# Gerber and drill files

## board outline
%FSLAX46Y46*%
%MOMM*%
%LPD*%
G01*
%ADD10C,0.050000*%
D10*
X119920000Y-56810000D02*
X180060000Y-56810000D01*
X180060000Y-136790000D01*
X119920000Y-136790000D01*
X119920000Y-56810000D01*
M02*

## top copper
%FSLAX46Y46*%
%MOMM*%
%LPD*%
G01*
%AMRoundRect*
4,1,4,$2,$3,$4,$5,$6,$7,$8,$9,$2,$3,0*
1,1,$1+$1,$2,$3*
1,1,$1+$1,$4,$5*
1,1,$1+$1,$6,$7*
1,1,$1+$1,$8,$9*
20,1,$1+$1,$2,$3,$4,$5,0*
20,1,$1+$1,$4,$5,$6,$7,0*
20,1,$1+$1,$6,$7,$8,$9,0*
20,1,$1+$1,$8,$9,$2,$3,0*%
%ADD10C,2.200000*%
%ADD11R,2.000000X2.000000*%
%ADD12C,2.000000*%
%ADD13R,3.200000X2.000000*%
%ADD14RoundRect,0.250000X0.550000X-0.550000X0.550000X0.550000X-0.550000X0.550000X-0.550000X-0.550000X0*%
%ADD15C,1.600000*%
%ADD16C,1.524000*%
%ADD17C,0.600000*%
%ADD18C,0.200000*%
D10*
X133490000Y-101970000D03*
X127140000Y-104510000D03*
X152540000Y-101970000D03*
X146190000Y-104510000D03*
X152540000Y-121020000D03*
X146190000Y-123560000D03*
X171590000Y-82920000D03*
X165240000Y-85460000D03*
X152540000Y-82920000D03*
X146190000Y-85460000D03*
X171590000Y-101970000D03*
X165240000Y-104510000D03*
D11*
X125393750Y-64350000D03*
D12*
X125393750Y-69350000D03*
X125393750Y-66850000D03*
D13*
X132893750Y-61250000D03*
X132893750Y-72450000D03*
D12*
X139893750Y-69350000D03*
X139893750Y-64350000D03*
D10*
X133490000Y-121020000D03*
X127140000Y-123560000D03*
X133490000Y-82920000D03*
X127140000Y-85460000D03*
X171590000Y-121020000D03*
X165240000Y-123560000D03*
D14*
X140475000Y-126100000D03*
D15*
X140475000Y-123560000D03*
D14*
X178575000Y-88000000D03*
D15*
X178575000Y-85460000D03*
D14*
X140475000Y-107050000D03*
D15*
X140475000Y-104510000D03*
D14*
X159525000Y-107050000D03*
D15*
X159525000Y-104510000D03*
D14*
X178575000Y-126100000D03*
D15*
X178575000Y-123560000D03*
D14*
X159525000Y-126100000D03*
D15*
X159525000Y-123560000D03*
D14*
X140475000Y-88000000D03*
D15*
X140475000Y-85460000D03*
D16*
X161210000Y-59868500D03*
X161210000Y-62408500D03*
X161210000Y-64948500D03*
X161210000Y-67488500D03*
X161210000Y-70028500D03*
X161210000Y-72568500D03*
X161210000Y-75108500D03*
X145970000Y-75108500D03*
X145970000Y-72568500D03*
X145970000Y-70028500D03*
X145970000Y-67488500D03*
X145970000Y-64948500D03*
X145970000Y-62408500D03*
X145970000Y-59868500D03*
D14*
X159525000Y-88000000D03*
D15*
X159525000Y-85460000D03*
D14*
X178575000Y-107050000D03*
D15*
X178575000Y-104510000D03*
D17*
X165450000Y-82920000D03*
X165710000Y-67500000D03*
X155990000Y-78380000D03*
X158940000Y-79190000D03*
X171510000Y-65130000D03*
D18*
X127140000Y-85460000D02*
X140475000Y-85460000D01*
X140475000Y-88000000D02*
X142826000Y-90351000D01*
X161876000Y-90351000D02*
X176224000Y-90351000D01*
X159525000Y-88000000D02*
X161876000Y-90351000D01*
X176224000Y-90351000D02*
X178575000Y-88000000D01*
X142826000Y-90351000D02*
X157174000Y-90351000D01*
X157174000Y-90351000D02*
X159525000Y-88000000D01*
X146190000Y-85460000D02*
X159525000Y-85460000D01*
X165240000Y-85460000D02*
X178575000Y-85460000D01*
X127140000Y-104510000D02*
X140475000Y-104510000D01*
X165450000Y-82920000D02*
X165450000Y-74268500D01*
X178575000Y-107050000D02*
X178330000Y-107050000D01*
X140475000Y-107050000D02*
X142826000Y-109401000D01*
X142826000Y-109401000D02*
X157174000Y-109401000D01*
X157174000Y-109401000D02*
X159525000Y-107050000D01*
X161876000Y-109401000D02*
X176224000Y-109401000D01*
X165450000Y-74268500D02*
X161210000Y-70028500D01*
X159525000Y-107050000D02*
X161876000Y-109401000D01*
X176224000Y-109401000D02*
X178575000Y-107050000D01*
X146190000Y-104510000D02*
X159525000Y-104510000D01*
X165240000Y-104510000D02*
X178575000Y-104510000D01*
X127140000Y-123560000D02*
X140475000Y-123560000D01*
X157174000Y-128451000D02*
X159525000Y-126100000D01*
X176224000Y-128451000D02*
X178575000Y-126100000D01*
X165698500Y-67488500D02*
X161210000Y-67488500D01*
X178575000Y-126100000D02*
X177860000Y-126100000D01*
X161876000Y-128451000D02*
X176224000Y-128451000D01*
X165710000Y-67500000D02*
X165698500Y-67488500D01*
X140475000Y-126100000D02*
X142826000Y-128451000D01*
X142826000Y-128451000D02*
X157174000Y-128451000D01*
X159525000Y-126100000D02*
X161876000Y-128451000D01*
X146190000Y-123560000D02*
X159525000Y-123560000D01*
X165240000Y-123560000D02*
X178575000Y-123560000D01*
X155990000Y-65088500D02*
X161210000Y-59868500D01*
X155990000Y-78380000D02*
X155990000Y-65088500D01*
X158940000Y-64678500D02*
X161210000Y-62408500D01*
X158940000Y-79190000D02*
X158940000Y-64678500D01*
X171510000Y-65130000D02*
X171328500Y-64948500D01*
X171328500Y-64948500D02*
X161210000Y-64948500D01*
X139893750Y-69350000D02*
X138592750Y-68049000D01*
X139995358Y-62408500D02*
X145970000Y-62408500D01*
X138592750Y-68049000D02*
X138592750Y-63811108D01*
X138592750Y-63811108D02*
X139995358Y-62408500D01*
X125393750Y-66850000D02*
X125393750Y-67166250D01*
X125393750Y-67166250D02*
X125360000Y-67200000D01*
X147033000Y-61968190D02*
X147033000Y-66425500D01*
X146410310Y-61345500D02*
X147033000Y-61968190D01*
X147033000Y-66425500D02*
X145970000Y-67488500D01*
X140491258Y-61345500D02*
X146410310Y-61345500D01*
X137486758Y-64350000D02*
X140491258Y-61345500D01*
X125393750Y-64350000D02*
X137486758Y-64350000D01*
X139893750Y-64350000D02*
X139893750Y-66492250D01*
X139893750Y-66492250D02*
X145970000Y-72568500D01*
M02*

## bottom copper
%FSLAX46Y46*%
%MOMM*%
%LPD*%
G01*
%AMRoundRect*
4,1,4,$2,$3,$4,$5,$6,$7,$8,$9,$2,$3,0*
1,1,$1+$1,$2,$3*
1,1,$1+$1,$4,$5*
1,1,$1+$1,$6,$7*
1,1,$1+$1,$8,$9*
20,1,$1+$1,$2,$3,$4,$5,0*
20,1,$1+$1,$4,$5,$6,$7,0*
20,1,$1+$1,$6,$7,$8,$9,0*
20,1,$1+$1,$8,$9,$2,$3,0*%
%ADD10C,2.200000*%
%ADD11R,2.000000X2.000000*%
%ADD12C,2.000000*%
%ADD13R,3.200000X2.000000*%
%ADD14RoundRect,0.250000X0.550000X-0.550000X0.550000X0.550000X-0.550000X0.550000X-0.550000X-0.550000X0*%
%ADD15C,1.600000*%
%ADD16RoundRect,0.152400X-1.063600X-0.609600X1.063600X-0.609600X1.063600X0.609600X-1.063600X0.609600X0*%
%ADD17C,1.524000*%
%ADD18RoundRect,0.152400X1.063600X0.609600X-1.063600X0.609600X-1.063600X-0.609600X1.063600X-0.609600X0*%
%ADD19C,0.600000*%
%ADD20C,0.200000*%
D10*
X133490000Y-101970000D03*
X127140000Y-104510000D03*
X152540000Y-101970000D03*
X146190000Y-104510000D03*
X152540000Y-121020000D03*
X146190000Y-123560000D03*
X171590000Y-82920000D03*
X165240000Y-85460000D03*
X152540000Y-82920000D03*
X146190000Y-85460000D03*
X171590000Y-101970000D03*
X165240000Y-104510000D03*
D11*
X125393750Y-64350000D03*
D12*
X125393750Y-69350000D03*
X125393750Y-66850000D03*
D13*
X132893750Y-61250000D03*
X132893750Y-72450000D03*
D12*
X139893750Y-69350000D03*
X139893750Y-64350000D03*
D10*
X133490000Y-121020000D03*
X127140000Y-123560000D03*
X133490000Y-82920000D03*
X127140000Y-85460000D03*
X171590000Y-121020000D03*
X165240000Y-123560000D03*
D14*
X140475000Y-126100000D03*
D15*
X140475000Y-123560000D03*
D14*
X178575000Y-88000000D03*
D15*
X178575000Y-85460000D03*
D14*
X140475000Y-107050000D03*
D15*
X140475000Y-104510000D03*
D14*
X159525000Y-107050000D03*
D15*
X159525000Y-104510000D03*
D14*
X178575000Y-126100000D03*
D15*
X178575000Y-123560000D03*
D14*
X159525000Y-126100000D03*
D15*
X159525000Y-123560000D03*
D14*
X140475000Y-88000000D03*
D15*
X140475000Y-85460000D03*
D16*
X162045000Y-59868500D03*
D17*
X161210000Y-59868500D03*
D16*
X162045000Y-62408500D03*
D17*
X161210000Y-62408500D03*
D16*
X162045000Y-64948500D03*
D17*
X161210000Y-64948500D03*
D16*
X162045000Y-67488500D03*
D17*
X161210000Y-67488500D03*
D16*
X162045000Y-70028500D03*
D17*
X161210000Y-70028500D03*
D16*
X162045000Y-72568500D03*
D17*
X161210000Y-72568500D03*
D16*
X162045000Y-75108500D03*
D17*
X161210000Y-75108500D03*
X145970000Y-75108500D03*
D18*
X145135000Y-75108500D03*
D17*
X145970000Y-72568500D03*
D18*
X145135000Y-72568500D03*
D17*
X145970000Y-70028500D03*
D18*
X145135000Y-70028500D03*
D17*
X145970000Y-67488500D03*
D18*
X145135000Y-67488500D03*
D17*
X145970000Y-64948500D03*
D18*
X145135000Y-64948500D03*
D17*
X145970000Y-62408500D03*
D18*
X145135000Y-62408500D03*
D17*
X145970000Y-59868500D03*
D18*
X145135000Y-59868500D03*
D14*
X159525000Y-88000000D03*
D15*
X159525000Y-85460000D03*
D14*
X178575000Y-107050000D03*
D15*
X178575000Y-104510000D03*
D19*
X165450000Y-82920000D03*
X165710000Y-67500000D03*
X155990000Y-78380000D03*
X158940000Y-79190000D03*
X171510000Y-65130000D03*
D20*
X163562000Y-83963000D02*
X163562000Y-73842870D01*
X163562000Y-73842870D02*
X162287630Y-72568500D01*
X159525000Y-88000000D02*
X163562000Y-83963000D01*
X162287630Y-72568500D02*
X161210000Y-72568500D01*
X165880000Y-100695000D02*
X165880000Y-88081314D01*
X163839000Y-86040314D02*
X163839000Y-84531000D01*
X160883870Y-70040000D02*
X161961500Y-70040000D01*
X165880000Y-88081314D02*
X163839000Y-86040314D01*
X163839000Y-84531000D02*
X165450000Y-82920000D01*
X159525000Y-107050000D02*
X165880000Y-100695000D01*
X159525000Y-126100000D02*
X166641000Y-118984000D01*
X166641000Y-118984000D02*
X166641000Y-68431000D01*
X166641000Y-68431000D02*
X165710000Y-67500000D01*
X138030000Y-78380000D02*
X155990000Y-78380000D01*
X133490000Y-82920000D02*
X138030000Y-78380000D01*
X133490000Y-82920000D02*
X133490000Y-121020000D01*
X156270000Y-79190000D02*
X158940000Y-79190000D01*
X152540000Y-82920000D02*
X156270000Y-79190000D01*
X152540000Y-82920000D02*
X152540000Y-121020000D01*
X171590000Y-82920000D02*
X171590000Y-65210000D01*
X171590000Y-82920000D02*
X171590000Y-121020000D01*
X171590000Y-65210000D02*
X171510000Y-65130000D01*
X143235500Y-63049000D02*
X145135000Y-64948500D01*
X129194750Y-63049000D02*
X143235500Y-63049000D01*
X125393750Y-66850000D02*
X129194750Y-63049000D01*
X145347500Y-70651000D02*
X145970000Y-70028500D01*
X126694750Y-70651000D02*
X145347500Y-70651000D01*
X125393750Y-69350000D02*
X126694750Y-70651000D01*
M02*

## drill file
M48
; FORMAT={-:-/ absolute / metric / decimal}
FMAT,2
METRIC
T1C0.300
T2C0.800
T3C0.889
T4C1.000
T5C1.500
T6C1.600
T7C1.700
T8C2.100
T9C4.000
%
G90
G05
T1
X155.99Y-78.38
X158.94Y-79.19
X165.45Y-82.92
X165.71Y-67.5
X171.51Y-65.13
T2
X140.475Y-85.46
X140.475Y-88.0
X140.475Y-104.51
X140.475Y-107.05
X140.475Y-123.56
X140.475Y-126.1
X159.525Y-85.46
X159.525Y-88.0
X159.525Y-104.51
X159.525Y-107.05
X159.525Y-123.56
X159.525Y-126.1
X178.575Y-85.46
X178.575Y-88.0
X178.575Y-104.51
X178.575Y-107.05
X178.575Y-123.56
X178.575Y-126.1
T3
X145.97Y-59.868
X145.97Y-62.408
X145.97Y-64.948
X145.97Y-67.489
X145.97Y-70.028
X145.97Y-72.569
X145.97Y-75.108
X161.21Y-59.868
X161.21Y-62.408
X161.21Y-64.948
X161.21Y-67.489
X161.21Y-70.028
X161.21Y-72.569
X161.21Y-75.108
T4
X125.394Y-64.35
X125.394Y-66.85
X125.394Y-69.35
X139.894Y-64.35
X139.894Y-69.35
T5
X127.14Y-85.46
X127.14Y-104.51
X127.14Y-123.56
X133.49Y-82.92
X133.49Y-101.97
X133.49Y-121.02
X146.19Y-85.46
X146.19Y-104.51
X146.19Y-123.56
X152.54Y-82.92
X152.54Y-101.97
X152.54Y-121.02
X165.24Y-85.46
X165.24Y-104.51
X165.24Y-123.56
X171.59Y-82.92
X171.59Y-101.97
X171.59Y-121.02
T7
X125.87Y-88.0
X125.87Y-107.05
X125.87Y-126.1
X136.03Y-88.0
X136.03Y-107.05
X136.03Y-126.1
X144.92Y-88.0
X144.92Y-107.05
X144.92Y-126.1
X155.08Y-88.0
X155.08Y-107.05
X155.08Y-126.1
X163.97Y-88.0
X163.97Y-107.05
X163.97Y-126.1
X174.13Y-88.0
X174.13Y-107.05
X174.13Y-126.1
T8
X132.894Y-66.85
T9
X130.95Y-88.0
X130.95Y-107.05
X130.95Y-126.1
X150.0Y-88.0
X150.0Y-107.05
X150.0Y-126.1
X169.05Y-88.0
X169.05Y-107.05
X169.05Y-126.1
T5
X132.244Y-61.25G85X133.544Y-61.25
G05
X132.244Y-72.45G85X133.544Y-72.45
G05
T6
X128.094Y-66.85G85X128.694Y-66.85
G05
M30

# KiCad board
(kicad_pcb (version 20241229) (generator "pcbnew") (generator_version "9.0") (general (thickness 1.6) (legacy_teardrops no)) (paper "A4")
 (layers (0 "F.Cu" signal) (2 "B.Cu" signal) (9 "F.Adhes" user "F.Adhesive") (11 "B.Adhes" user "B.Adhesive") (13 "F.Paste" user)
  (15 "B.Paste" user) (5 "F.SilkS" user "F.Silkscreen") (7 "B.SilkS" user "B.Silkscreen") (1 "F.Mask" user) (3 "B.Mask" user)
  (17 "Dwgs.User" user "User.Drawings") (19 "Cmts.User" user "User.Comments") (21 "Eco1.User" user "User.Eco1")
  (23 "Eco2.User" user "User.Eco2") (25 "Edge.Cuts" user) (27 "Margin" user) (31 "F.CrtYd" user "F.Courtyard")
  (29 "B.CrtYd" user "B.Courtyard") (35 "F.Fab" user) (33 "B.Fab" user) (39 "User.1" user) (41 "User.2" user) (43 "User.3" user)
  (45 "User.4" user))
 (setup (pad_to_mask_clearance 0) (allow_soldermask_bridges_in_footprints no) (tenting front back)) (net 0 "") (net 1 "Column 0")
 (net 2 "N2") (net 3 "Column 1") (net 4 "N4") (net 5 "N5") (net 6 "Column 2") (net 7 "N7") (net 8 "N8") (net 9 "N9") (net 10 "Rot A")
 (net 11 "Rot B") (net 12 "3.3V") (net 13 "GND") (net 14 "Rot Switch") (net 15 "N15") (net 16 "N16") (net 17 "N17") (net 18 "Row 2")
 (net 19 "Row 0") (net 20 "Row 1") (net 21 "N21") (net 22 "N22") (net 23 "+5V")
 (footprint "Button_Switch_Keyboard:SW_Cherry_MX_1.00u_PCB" (layer "F.Cu") (at 133.49 101.97)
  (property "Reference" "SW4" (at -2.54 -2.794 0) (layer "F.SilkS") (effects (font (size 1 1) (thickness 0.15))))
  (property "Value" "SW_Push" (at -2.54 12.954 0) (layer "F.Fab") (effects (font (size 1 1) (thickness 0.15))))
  (pad "" np_thru_hole circle (at -7.62 5.08) (size 1.7 1.7) (drill 1.7) (layers "*.Cu" "*.Mask"))
  (pad "" np_thru_hole circle (at -2.54 5.08) (size 4 4) (drill 4) (layers "*.Cu" "*.Mask"))
  (pad "" np_thru_hole circle (at 2.54 5.08) (size 1.7 1.7) (drill 1.7) (layers "*.Cu" "*.Mask"))
  (pad "1" thru_hole circle (at 0 0) (size 2.2 2.2) (drill 1.5) (layers "*.Cu" "*.Mask") (remove_unused_layers no) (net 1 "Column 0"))
  (pad "2" thru_hole circle (at -6.35 2.54) (size 2.2 2.2) (drill 1.5) (layers "*.Cu" "*.Mask") (remove_unused_layers no) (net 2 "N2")))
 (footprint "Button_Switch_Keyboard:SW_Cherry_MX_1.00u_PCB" (layer "F.Cu") (at 152.54 101.97)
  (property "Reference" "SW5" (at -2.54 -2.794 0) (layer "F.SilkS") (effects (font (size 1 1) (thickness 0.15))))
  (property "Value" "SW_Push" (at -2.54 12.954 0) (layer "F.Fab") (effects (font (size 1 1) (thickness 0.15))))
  (pad "" np_thru_hole circle (at -7.62 5.08) (size 1.7 1.7) (drill 1.7) (layers "*.Cu" "*.Mask"))
  (pad "" np_thru_hole circle (at -2.54 5.08) (size 4 4) (drill 4) (layers "*.Cu" "*.Mask"))
  (pad "" np_thru_hole circle (at 2.54 5.08) (size 1.7 1.7) (drill 1.7) (layers "*.Cu" "*.Mask"))
  (pad "1" thru_hole circle (at 0 0) (size 2.2 2.2) (drill 1.5) (layers "*.Cu" "*.Mask") (remove_unused_layers no) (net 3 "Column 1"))
  (pad "2" thru_hole circle (at -6.35 2.54) (size 2.2 2.2) (drill 1.5) (layers "*.Cu" "*.Mask") (remove_unused_layers no) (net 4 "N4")))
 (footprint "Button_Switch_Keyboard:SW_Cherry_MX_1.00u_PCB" (layer "F.Cu") (at 152.54 121.02)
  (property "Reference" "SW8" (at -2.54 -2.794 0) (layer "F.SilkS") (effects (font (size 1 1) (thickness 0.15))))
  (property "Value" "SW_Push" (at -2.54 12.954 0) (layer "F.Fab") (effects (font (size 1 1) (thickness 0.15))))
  (pad "" np_thru_hole circle (at -7.62 5.08) (size 1.7 1.7) (drill 1.7) (layers "*.Cu" "*.Mask"))
  (pad "" np_thru_hole circle (at -2.54 5.08) (size 4 4) (drill 4) (layers "*.Cu" "*.Mask"))
  (pad "" np_thru_hole circle (at 2.54 5.08) (size 1.7 1.7) (drill 1.7) (layers "*.Cu" "*.Mask"))
  (pad "1" thru_hole circle (at 0 0) (size 2.2 2.2) (drill 1.5) (layers "*.Cu" "*.Mask") (remove_unused_layers no) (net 3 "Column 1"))
  (pad "2" thru_hole circle (at -6.35 2.54) (size 2.2 2.2) (drill 1.5) (layers "*.Cu" "*.Mask") (remove_unused_layers no) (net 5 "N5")))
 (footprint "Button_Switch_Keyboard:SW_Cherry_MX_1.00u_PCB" (layer "F.Cu") (at 171.59 82.92)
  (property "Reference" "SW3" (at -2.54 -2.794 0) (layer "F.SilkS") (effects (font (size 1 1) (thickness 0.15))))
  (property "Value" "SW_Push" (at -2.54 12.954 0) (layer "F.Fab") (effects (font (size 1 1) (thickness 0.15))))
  (pad "" np_thru_hole circle (at -7.62 5.08) (size 1.7 1.7) (drill 1.7) (layers "*.Cu" "*.Mask"))
  (pad "" np_thru_hole circle (at -2.54 5.08) (size 4 4) (drill 4) (layers "*.Cu" "*.Mask"))
  (pad "" np_thru_hole circle (at 2.54 5.08) (size 1.7 1.7) (drill 1.7) (layers "*.Cu" "*.Mask"))
  (pad "1" thru_hole circle (at 0 0) (size 2.2 2.2) (drill 1.5) (layers "*.Cu" "*.Mask") (remove_unused_layers no) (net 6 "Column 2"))
  (pad "2" thru_hole circle (at -6.35 2.54) (size 2.2 2.2) (drill 1.5) (layers "*.Cu" "*.Mask") (remove_unused_layers no) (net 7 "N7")))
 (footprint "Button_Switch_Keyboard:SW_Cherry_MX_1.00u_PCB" (layer "F.Cu") (at 152.54 82.92)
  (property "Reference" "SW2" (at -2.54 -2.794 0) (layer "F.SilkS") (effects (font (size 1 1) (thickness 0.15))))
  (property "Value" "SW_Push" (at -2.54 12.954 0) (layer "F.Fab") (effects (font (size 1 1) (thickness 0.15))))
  (pad "" np_thru_hole circle (at -7.62 5.08) (size 1.7 1.7) (drill 1.7) (layers "*.Cu" "*.Mask"))
  (pad "" np_thru_hole circle (at -2.54 5.08) (size 4 4) (drill 4) (layers "*.Cu" "*.Mask"))
  (pad "" np_thru_hole circle (at 2.54 5.08) (size 1.7 1.7) (drill 1.7) (layers "*.Cu" "*.Mask"))
  (pad "1" thru_hole circle (at 0 0) (size 2.2 2.2) (drill 1.5) (layers "*.Cu" "*.Mask") (remove_unused_layers no) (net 3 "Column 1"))
  (pad "2" thru_hole circle (at -6.35 2.54) (size 2.2 2.2) (drill 1.5) (layers "*.Cu" "*.Mask") (remove_unused_layers no) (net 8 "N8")))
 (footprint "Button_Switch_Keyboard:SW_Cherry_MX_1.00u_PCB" (layer "F.Cu") (at 171.59 101.97)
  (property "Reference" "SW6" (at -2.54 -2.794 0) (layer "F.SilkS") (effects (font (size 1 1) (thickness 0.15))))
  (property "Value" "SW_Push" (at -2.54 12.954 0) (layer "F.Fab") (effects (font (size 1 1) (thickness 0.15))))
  (pad "" np_thru_hole circle (at -7.62 5.08) (size 1.7 1.7) (drill 1.7) (layers "*.Cu" "*.Mask"))
  (pad "" np_thru_hole circle (at -2.54 5.08) (size 4 4) (drill 4) (layers "*.Cu" "*.Mask"))
  (pad "" np_thru_hole circle (at 2.54 5.08) (size 1.7 1.7) (drill 1.7) (layers "*.Cu" "*.Mask"))
  (pad "1" thru_hole circle (at 0 0) (size 2.2 2.2) (drill 1.5) (layers "*.Cu" "*.Mask") (remove_unused_layers no) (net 6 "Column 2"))
  (pad "2" thru_hole circle (at -6.35 2.54) (size 2.2 2.2) (drill 1.5) (layers "*.Cu" "*.Mask") (remove_unused_layers no) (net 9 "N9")))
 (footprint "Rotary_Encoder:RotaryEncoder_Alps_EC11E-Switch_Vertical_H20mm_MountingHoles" (layer "F.Cu") (at 125.39375 64.35)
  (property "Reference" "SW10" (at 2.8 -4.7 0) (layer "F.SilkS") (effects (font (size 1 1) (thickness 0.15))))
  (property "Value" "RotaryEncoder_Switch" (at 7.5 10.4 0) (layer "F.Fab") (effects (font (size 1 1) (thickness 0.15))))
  (pad "" np_thru_hole oval (at 3 2.5) (size 2.2 1.6) (drill oval 2.2 1.6) (layers "*.Mask"))
  (pad "" np_thru_hole circle (at 7.5 2.5) (size 2.1 2.1) (drill 2.1) (layers "*.Mask"))
  (pad "A" thru_hole rect (at 0 0) (size 2 2) (drill 1) (layers "*.Cu" "*.Mask") (remove_unused_layers no) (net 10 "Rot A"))
  (pad "B" thru_hole circle (at 0 5) (size 2 2) (drill 1) (layers "*.Cu" "*.Mask") (remove_unused_layers no) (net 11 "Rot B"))
  (pad "C" thru_hole circle (at 0 2.5) (size 2 2) (drill 1) (layers "*.Cu" "*.Mask") (remove_unused_layers no) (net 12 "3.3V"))
  (pad "MP" thru_hole rect (at 7.5 -3.1) (size 3.2 2) (drill oval 2.8 1.5) (layers "*.Cu" "*.Mask") (remove_unused_layers no))
  (pad "MP" thru_hole rect (at 7.5 8.1) (size 3.2 2) (drill oval 2.8 1.5) (layers "*.Cu" "*.Mask") (remove_unused_layers no))
  (pad "S1" thru_hole circle (at 14.5 5) (size 2 2) (drill 1) (layers "*.Cu" "*.Mask") (remove_unused_layers no) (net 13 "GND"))
  (pad "S2" thru_hole circle (at 14.5 0) (size 2 2) (drill 1) (layers "*.Cu" "*.Mask") (remove_unused_layers no) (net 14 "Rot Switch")))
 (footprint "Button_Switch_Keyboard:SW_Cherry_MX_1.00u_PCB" (layer "F.Cu") (at 133.49 121.02)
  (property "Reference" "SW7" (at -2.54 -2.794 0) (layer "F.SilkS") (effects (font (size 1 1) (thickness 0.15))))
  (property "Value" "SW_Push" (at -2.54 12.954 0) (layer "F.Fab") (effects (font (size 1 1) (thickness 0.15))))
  (pad "" np_thru_hole circle (at -7.62 5.08) (size 1.7 1.7) (drill 1.7) (layers "*.Cu" "*.Mask"))
  (pad "" np_thru_hole circle (at -2.54 5.08) (size 4 4) (drill 4) (layers "*.Cu" "*.Mask"))
  (pad "" np_thru_hole circle (at 2.54 5.08) (size 1.7 1.7) (drill 1.7) (layers "*.Cu" "*.Mask"))
  (pad "1" thru_hole circle (at 0 0) (size 2.2 2.2) (drill 1.5) (layers "*.Cu" "*.Mask") (remove_unused_layers no) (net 1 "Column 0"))
  (pad "2" thru_hole circle (at -6.35 2.54) (size 2.2 2.2) (drill 1.5) (layers "*.Cu" "*.Mask") (remove_unused_layers no) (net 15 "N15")))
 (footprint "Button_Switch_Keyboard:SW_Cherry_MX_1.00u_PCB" (layer "F.Cu") (at 133.49 82.92)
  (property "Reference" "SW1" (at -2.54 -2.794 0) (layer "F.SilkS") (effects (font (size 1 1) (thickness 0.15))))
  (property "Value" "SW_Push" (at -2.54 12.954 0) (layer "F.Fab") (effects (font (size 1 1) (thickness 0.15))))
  (pad "" np_thru_hole circle (at -7.62 5.08) (size 1.7 1.7) (drill 1.7) (layers "*.Cu" "*.Mask"))
  (pad "" np_thru_hole circle (at -2.54 5.08) (size 4 4) (drill 4) (layers "*.Cu" "*.Mask"))
  (pad "" np_thru_hole circle (at 2.54 5.08) (size 1.7 1.7) (drill 1.7) (layers "*.Cu" "*.Mask"))
  (pad "1" thru_hole circle (at 0 0) (size 2.2 2.2) (drill 1.5) (layers "*.Cu" "*.Mask") (remove_unused_layers no) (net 1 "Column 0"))
  (pad "2" thru_hole circle (at -6.35 2.54) (size 2.2 2.2) (drill 1.5) (layers "*.Cu" "*.Mask") (remove_unused_layers no) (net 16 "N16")))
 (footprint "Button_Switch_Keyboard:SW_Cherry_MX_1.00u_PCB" (layer "F.Cu") (at 171.59 121.02)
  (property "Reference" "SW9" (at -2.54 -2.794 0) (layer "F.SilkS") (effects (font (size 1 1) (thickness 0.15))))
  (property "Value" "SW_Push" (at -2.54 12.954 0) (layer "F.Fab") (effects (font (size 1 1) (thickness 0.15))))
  (pad "" np_thru_hole circle (at -7.62 5.08) (size 1.7 1.7) (drill 1.7) (layers "*.Cu" "*.Mask"))
  (pad "" np_thru_hole circle (at -2.54 5.08) (size 4 4) (drill 4) (layers "*.Cu" "*.Mask"))
  (pad "" np_thru_hole circle (at 2.54 5.08) (size 1.7 1.7) (drill 1.7) (layers "*.Cu" "*.Mask"))
  (pad "1" thru_hole circle (at 0 0) (size 2.2 2.2) (drill 1.5) (layers "*.Cu" "*.Mask") (remove_unused_layers no) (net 6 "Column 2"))
  (pad "2" thru_hole circle (at -6.35 2.54) (size 2.2 2.2) (drill 1.5) (layers "*.Cu" "*.Mask") (remove_unused_layers no) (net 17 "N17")))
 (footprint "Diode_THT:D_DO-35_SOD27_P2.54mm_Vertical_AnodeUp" (layer "B.Cu") (at 140.475 126.1 90)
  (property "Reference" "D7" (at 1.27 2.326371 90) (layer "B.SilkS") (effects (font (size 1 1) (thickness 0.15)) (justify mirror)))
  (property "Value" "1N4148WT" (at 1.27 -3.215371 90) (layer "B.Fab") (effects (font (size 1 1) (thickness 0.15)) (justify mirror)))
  (pad "1" thru_hole roundrect (at 0 0 90) (size 1.6 1.6) (drill 0.8) (layers "*.Cu" "*.Mask") (remove_unused_layers no)
   (roundrect_rratio 0.15625) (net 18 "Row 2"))
  (pad "2" thru_hole circle (at 2.54 0 90) (size 1.6 1.6) (drill 0.8) (layers "*.Cu" "*.Mask") (remove_unused_layers no) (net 15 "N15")))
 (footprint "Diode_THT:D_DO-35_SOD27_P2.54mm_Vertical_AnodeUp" (layer "B.Cu") (at 178.575 88 90)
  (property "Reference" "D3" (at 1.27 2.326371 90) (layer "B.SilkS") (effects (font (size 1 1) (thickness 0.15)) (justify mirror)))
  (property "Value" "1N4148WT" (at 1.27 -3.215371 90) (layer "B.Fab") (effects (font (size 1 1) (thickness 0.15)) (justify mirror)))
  (pad "1" thru_hole roundrect (at 0 0 90) (size 1.6 1.6) (drill 0.8) (layers "*.Cu" "*.Mask") (remove_unused_layers no)
   (roundrect_rratio 0.15625) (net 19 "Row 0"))
  (pad "2" thru_hole circle (at 2.54 0 90) (size 1.6 1.6) (drill 0.8) (layers "*.Cu" "*.Mask") (remove_unused_layers no) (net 7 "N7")))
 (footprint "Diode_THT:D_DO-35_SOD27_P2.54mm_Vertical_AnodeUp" (layer "B.Cu") (at 140.475 107.05 90)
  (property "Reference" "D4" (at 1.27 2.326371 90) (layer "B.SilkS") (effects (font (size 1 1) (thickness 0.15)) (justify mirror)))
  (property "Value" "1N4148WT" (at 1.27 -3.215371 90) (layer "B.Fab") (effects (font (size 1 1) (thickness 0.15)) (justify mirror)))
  (pad "1" thru_hole roundrect (at 0 0 90) (size 1.6 1.6) (drill 0.8) (layers "*.Cu" "*.Mask") (remove_unused_layers no)
   (roundrect_rratio 0.15625) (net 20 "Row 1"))
  (pad "2" thru_hole circle (at 2.54 0 90) (size 1.6 1.6) (drill 0.8) (layers "*.Cu" "*.Mask") (remove_unused_layers no) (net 2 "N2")))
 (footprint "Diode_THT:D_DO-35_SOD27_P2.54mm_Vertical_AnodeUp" (layer "B.Cu") (at 159.525 107.05 90)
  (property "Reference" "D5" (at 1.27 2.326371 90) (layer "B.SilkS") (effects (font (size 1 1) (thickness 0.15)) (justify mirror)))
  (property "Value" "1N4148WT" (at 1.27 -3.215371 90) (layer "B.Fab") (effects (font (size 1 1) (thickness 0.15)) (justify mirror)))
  (pad "1" thru_hole roundrect (at 0 0 90) (size 1.6 1.6) (drill 0.8) (layers "*.Cu" "*.Mask") (remove_unused_layers no)
   (roundrect_rratio 0.15625) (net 20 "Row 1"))
  (pad "2" thru_hole circle (at 2.54 0 90) (size 1.6 1.6) (drill 0.8) (layers "*.Cu" "*.Mask") (remove_unused_layers no) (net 4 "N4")))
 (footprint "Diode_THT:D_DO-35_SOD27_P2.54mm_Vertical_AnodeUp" (layer "B.Cu") (at 178.575 126.1 90)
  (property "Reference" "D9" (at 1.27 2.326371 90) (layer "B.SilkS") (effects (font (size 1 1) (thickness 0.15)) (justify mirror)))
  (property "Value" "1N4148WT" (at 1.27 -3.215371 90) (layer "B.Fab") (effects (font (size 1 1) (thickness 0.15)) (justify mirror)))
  (pad "1" thru_hole roundrect (at 0 0 90) (size 1.6 1.6) (drill 0.8) (layers "*.Cu" "*.Mask") (remove_unused_layers no)
   (roundrect_rratio 0.15625) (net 18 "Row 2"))
  (pad "2" thru_hole circle (at 2.54 0 90) (size 1.6 1.6) (drill 0.8) (layers "*.Cu" "*.Mask") (remove_unused_layers no) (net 17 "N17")))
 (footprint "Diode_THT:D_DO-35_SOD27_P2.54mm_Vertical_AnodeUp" (layer "B.Cu") (at 159.525 126.1 90)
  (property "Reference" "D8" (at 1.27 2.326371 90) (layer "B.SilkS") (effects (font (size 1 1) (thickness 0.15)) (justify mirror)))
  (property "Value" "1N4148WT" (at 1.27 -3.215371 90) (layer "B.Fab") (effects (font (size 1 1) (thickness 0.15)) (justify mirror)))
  (pad "1" thru_hole roundrect (at 0 0 90) (size 1.6 1.6) (drill 0.8) (layers "*.Cu" "*.Mask") (remove_unused_layers no)
   (roundrect_rratio 0.15625) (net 18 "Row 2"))
  (pad "2" thru_hole circle (at 2.54 0 90) (size 1.6 1.6) (drill 0.8) (layers "*.Cu" "*.Mask") (remove_unused_layers no) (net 5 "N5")))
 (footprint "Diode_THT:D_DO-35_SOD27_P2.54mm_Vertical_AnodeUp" (layer "B.Cu") (at 140.475 88 90)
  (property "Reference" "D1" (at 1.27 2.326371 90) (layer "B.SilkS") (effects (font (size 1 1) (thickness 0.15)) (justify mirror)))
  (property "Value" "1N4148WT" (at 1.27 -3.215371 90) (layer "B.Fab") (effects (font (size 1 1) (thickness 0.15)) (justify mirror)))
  (pad "1" thru_hole roundrect (at 0 0 90) (size 1.6 1.6) (drill 0.8) (layers "*.Cu" "*.Mask") (remove_unused_layers no)
   (roundrect_rratio 0.15625) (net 19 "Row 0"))
  (pad "2" thru_hole circle (at 2.54 0 90) (size 1.6 1.6) (drill 0.8) (layers "*.Cu" "*.Mask") (remove_unused_layers no) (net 16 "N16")))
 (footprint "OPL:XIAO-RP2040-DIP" (layer "B.Cu") (at 153.59 67.4885 180)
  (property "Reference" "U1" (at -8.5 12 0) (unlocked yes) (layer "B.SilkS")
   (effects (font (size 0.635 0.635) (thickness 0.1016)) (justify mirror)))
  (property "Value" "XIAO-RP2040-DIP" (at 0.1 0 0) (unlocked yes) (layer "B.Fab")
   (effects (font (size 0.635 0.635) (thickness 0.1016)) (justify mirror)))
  (pad "1" smd roundrect (at -8.455 7.62) (size 2.432 1.524) (layers "B.Cu" "B.Mask") (roundrect_rratio 0.1) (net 1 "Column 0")
   (thermal_bridge_angle 45))
  (pad "1" thru_hole circle (at -7.62 7.62) (size 1.524 1.524) (drill 0.889) (layers "*.Cu" "*.Mask") (remove_unused_layers no)
   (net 1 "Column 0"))
  (pad "2" smd roundrect (at -8.455 5.08) (size 2.432 1.524) (layers "B.Cu" "B.Mask") (roundrect_rratio 0.1) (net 3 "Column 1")
   (thermal_bridge_angle 45))
  (pad "2" thru_hole circle (at -7.62 5.08) (size 1.524 1.524) (drill 0.889) (layers "*.Cu" "*.Mask") (remove_unused_layers no)
   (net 3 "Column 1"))
  (pad "3" smd roundrect (at -8.455 2.54) (size 2.432 1.524) (layers "B.Cu" "B.Mask") (roundrect_rratio 0.1) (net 6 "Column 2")
   (thermal_bridge_angle 45))
  (pad "3" thru_hole circle (at -7.62 2.54) (size 1.524 1.524) (drill 0.889) (layers "*.Cu" "*.Mask") (remove_unused_layers no)
   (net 6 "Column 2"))
  (pad "4" smd roundrect (at -8.455 0) (size 2.432 1.524) (layers "B.Cu" "B.Mask") (roundrect_rratio 0.1) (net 18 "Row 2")
   (thermal_bridge_angle 45))
  (pad "4" thru_hole circle (at -7.62 0) (size 1.524 1.524) (drill 0.889) (layers "*.Cu" "*.Mask") (remove_unused_layers no)
   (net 18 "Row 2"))
  (pad "5" smd roundrect (at -8.455 -2.54) (size 2.432 1.524) (layers "B.Cu" "B.Mask") (roundrect_rratio 0.1) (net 20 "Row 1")
   (thermal_bridge_angle 45))
  (pad "5" thru_hole circle (at -7.62 -2.54) (size 1.524 1.524) (drill 0.889) (layers "*.Cu" "*.Mask") (remove_unused_layers no)
   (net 20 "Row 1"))
  (pad "6" smd roundrect (at -8.455 -5.08) (size 2.432 1.524) (layers "B.Cu" "B.Mask") (roundrect_rratio 0.1) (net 19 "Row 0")
   (thermal_bridge_angle 45))
  (pad "6" thru_hole circle (at -7.62 -5.08) (size 1.524 1.524) (drill 0.889) (layers "*.Cu" "*.Mask") (remove_unused_layers no)
   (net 19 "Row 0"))
  (pad "7" smd roundrect (at -8.455 -7.62) (size 2.432 1.524) (layers "B.Cu" "B.Mask") (roundrect_rratio 0.1) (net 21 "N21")
   (thermal_bridge_angle 45))
  (pad "7" thru_hole circle (at -7.62 -7.62) (size 1.524 1.524) (drill 0.889) (layers "*.Cu" "*.Mask") (remove_unused_layers no)
   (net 21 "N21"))
  (pad "8" thru_hole circle (at 7.62 -7.62 180) (size 1.524 1.524) (drill 0.889) (layers "*.Cu" "*.Mask") (remove_unused_layers no)
   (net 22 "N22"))
  (pad "8" smd roundrect (at 8.455 -7.62 180) (size 2.432 1.524) (layers "B.Cu" "B.Mask") (roundrect_rratio 0.1) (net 22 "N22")
   (thermal_bridge_angle 45))
  (pad "9" thru_hole circle (at 7.62 -5.08 180) (size 1.524 1.524) (drill 0.889) (layers "*.Cu" "*.Mask") (remove_unused_layers no)
   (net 14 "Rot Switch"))
  (pad "9" smd roundrect (at 8.455 -5.08 180) (size 2.432 1.524) (layers "B.Cu" "B.Mask") (roundrect_rratio 0.1) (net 14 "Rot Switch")
   (thermal_bridge_angle 45))
  (pad "10" thru_hole circle (at 7.62 -2.54 180) (size 1.524 1.524) (drill 0.889) (layers "*.Cu" "*.Mask") (remove_unused_layers no)
   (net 11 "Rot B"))
  (pad "10" smd roundrect (at 8.455 -2.54 180) (size 2.432 1.524) (layers "B.Cu" "B.Mask") (roundrect_rratio 0.1) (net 11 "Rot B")
   (thermal_bridge_angle 45))
  (pad "11" thru_hole circle (at 7.62 0 180) (size 1.524 1.524) (drill 0.889) (layers "*.Cu" "*.Mask") (remove_unused_layers no)
   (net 10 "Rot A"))
  (pad "11" smd roundrect (at 8.455 0 180) (size 2.432 1.524) (layers "B.Cu" "B.Mask") (roundrect_rratio 0.1) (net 10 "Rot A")
   (thermal_bridge_angle 45))
  (pad "12" thru_hole circle (at 7.62 2.54 180) (size 1.524 1.524) (drill 0.889) (layers "*.Cu" "*.Mask") (remove_unused_layers no)
   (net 12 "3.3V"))
  (pad "12" smd roundrect (at 8.455 2.54 180) (size 2.432 1.524) (layers "B.Cu" "B.Mask") (roundrect_rratio 0.1) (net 12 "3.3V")
   (thermal_bridge_angle 45))
  (pad "13" thru_hole circle (at 7.62 5.08 180) (size 1.524 1.524) (drill 0.889) (layers "*.Cu" "*.Mask") (remove_unused_layers no)
   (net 13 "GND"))
  (pad "13" smd roundrect (at 8.455 5.08 180) (size 2.432 1.524) (layers "B.Cu" "B.Mask") (roundrect_rratio 0.1) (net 13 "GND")
   (thermal_bridge_angle 45))
  (pad "14" thru_hole circle (at 7.62 7.62 180) (size 1.524 1.524) (drill 0.889) (layers "*.Cu" "*.Mask") (remove_unused_layers no)
   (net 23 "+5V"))
  (pad "14" smd roundrect (at 8.455 7.62 180) (size 2.432 1.524) (layers "B.Cu" "B.Mask") (roundrect_rratio 0.1) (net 23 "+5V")
   (thermal_bridge_angle 45)))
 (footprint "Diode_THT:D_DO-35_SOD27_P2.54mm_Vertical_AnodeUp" (layer "B.Cu") (at 159.525 88 90)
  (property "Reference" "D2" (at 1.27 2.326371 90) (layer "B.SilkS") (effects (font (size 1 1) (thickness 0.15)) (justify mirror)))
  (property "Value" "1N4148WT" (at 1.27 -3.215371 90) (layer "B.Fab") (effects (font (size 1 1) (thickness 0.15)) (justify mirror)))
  (pad "1" thru_hole roundrect (at 0 0 90) (size 1.6 1.6) (drill 0.8) (layers "*.Cu" "*.Mask") (remove_unused_layers no)
   (roundrect_rratio 0.15625) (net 19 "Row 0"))
  (pad "2" thru_hole circle (at 2.54 0 90) (size 1.6 1.6) (drill 0.8) (layers "*.Cu" "*.Mask") (remove_unused_layers no) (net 8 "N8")))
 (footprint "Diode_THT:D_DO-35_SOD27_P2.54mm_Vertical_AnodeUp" (layer "B.Cu") (at 178.575 107.05 90)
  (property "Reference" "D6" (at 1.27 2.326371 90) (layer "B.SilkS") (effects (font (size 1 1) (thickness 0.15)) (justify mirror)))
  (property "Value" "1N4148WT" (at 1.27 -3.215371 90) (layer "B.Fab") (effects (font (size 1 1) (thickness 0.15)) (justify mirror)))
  (pad "1" thru_hole roundrect (at 0 0 90) (size 1.6 1.6) (drill 0.8) (layers "*.Cu" "*.Mask") (remove_unused_layers no)
   (roundrect_rratio 0.15625) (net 20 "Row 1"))
  (pad "2" thru_hole circle (at 2.54 0 90) (size 1.6 1.6) (drill 0.8) (layers "*.Cu" "*.Mask") (remove_unused_layers no) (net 9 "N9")))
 (gr_rect (start 119.92 56.81) (end 180.06 136.79) (stroke (width 0.05) (type default)) (fill no) (layer "Edge.Cuts"))
 (segment (start 127.14 85.46) (end 140.475 85.46) (width 0.2) (layer "F.Cu") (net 16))
 (segment (start 140.475 88) (end 142.826 90.351) (width 0.2) (layer "F.Cu") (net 19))
 (segment (start 161.876 90.351) (end 176.224 90.351) (width 0.2) (layer "F.Cu") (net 19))
 (segment (start 159.525 88) (end 161.876 90.351) (width 0.2) (layer "F.Cu") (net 19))
 (segment (start 176.224 90.351) (end 178.575 88) (width 0.2) (layer "F.Cu") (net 19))
 (segment (start 142.826 90.351) (end 157.174 90.351) (width 0.2) (layer "F.Cu") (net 19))
 (segment (start 157.174 90.351) (end 159.525 88) (width 0.2) (layer "F.Cu") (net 19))
 (segment (start 163.562 83.963) (end 163.562 73.84287) (width 0.2) (layer "B.Cu") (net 19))
 (segment (start 163.562 73.84287) (end 162.28763 72.5685) (width 0.2) (layer "B.Cu") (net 19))
 (segment (start 159.525 88) (end 163.562 83.963) (width 0.2) (layer "B.Cu") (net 19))
 (segment (start 162.28763 72.5685) (end 161.21 72.5685) (width 0.2) (layer "B.Cu") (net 19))
 (segment (start 146.19 85.46) (end 159.525 85.46) (width 0.2) (layer "F.Cu") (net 8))
 (segment (start 165.24 85.46) (end 178.575 85.46) (width 0.2) (layer "F.Cu") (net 7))
 (segment (start 127.14 104.51) (end 140.475 104.51) (width 0.2) (layer "F.Cu") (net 2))
 (segment (start 165.45 82.92) (end 165.45 74.2685) (width 0.2) (layer "F.Cu") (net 20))
 (segment (start 178.575 107.05) (end 178.33 107.05) (width 0.2) (layer "F.Cu") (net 20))
 (segment (start 140.475 107.05) (end 142.826 109.401) (width 0.2) (layer "F.Cu") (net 20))
 (segment (start 142.826 109.401) (end 157.174 109.401) (width 0.2) (layer "F.Cu") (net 20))
 (segment (start 157.174 109.401) (end 159.525 107.05) (width 0.2) (layer "F.Cu") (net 20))
 (segment (start 161.876 109.401) (end 176.224 109.401) (width 0.2) (layer "F.Cu") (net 20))
 (segment (start 165.45 74.2685) (end 161.21 70.0285) (width 0.2) (layer "F.Cu") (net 20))
 (segment (start 159.525 107.05) (end 161.876 109.401) (width 0.2) (layer "F.Cu") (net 20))
 (segment (start 176.224 109.401) (end 178.575 107.05) (width 0.2) (layer "F.Cu") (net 20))
 (via (at 165.45 82.92) (size 0.6) (drill 0.3) (layers "F.Cu" "B.Cu") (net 20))
 (segment (start 165.88 100.695) (end 165.88 88.081314) (width 0.2) (layer "B.Cu") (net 20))
 (segment (start 163.839 86.040314) (end 163.839 84.531) (width 0.2) (layer "B.Cu") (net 20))
 (segment (start 160.88387 70.04) (end 161.9615 70.04) (width 0.2) (layer "B.Cu") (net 20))
 (segment (start 165.88 88.081314) (end 163.839 86.040314) (width 0.2) (layer "B.Cu") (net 20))
 (segment (start 163.839 84.531) (end 165.45 82.92) (width 0.2) (layer "B.Cu") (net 20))
 (segment (start 159.525 107.05) (end 165.88 100.695) (width 0.2) (layer "B.Cu") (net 20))
 (segment (start 146.19 104.51) (end 159.525 104.51) (width 0.2) (layer "F.Cu") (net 4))
 (segment (start 165.24 104.51) (end 178.575 104.51) (width 0.2) (layer "F.Cu") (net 9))
 (segment (start 127.14 123.56) (end 140.475 123.56) (width 0.2) (layer "F.Cu") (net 15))
 (segment (start 157.174 128.451) (end 159.525 126.1) (width 0.2) (layer "F.Cu") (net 18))
 (segment (start 176.224 128.451) (end 178.575 126.1) (width 0.2) (layer "F.Cu") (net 18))
 (segment (start 165.6985 67.4885) (end 161.21 67.4885) (width 0.2) (layer "F.Cu") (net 18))
 (segment (start 178.575 126.1) (end 177.86 126.1) (width 0.2) (layer "F.Cu") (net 18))
 (segment (start 161.876 128.451) (end 176.224 128.451) (width 0.2) (layer "F.Cu") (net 18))
 (segment (start 165.71 67.5) (end 165.6985 67.4885) (width 0.2) (layer "F.Cu") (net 18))
 (segment (start 140.475 126.1) (end 142.826 128.451) (width 0.2) (layer "F.Cu") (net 18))
 (segment (start 142.826 128.451) (end 157.174 128.451) (width 0.2) (layer "F.Cu") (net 18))
 (segment (start 159.525 126.1) (end 161.876 128.451) (width 0.2) (layer "F.Cu") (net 18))
 (via (at 165.71 67.5) (size 0.6) (drill 0.3) (layers "F.Cu" "B.Cu") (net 18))
 (segment (start 159.525 126.1) (end 166.641 118.984) (width 0.2) (layer "B.Cu") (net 18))
 (segment (start 166.641 118.984) (end 166.641 68.431) (width 0.2) (layer "B.Cu") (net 18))
 (segment (start 166.641 68.431) (end 165.71 67.5) (width 0.2) (layer "B.Cu") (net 18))
 (segment (start 146.19 123.56) (end 159.525 123.56) (width 0.2) (layer "F.Cu") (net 5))
 (segment (start 165.24 123.56) (end 178.575 123.56) (width 0.2) (layer "F.Cu") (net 17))
 (segment (start 155.99 65.0885) (end 161.21 59.8685) (width 0.2) (layer "F.Cu") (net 1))
 (segment (start 155.99 78.38) (end 155.99 65.0885) (width 0.2) (layer "F.Cu") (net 1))
 (via (at 155.99 78.38) (size 0.6) (drill 0.3) (layers "F.Cu" "B.Cu") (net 1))
 (segment (start 138.03 78.38) (end 155.99 78.38) (width 0.2) (layer "B.Cu") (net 1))
 (segment (start 133.49 82.92) (end 138.03 78.38) (width 0.2) (layer "B.Cu") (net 1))
 (segment (start 133.49 82.92) (end 133.49 121.02) (width 0.2) (layer "B.Cu") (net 1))
 (segment (start 158.94 64.6785) (end 161.21 62.4085) (width 0.2) (layer "F.Cu") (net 3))
 (segment (start 158.94 79.19) (end 158.94 64.6785) (width 0.2) (layer "F.Cu") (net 3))
 (via (at 158.94 79.19) (size 0.6) (drill 0.3) (layers "F.Cu" "B.Cu") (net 3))
 (segment (start 156.27 79.19) (end 158.94 79.19) (width 0.2) (layer "B.Cu") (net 3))
 (segment (start 152.54 82.92) (end 156.27 79.19) (width 0.2) (layer "B.Cu") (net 3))
 (segment (start 152.54 82.92) (end 152.54 121.02) (width 0.2) (layer "B.Cu") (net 3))
 (segment (start 171.51 65.13) (end 171.3285 64.9485) (width 0.2) (layer "F.Cu") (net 6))
 (segment (start 171.3285 64.9485) (end 161.21 64.9485) (width 0.2) (layer "F.Cu") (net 6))
 (via (at 171.51 65.13) (size 0.6) (drill 0.3) (layers "F.Cu" "B.Cu") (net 6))
 (segment (start 171.59 82.92) (end 171.59 65.21) (width 0.2) (layer "B.Cu") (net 6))
 (segment (start 171.59 82.92) (end 171.59 121.02) (width 0.2) (layer "B.Cu") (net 6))
 (segment (start 171.59 65.21) (end 171.51 65.13) (width 0.2) (layer "B.Cu") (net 6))
 (segment (start 139.89375 69.35) (end 138.59275 68.049) (width 0.2) (layer "F.Cu") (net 13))
 (segment (start 139.995358 62.4085) (end 145.97 62.4085) (width 0.2) (layer "F.Cu") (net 13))
 (segment (start 138.59275 68.049) (end 138.59275 63.811108) (width 0.2) (layer "F.Cu") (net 13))
 (segment (start 138.59275 63.811108) (end 139.995358 62.4085) (width 0.2) (layer "F.Cu") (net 13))
 (segment (start 125.39375 66.85) (end 125.39375 67.16625) (width 0.2) (layer "F.Cu") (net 12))
 (segment (start 125.39375 67.16625) (end 125.36 67.2) (width 0.2) (layer "F.Cu") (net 12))
 (segment (start 143.2355 63.049) (end 145.135 64.9485) (width 0.2) (layer "B.Cu") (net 12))
 (segment (start 129.19475 63.049) (end 143.2355 63.049) (width 0.2) (layer "B.Cu") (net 12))
 (segment (start 125.39375 66.85) (end 129.19475 63.049) (width 0.2) (layer "B.Cu") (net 12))
 (segment (start 145.3475 70.651) (end 145.97 70.0285) (width 0.2) (layer "B.Cu") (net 11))
 (segment (start 126.69475 70.651) (end 145.3475 70.651) (width 0.2) (layer "B.Cu") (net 11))
 (segment (start 125.39375 69.35) (end 126.69475 70.651) (width 0.2) (layer "B.Cu") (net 11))
 (segment (start 147.033 61.96819) (end 147.033 66.4255) (width 0.2) (layer "F.Cu") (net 10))
 (segment (start 146.41031 61.3455) (end 147.033 61.96819) (width 0.2) (layer "F.Cu") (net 10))
 (segment (start 147.033 66.4255) (end 145.97 67.4885) (width 0.2) (layer "F.Cu") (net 10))
 (segment (start 140.491258 61.3455) (end 146.41031 61.3455) (width 0.2) (layer "F.Cu") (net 10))
 (segment (start 137.486758 64.35) (end 140.491258 61.3455) (width 0.2) (layer "F.Cu") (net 10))
 (segment (start 125.39375 64.35) (end 137.486758 64.35) (width 0.2) (layer "F.Cu") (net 10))
 (segment (start 139.89375 64.35) (end 139.89375 66.49225) (width 0.2) (layer "F.Cu") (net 14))
 (segment (start 139.89375 66.49225) (end 145.97 72.5685) (width 0.2) (layer "F.Cu") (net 14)))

